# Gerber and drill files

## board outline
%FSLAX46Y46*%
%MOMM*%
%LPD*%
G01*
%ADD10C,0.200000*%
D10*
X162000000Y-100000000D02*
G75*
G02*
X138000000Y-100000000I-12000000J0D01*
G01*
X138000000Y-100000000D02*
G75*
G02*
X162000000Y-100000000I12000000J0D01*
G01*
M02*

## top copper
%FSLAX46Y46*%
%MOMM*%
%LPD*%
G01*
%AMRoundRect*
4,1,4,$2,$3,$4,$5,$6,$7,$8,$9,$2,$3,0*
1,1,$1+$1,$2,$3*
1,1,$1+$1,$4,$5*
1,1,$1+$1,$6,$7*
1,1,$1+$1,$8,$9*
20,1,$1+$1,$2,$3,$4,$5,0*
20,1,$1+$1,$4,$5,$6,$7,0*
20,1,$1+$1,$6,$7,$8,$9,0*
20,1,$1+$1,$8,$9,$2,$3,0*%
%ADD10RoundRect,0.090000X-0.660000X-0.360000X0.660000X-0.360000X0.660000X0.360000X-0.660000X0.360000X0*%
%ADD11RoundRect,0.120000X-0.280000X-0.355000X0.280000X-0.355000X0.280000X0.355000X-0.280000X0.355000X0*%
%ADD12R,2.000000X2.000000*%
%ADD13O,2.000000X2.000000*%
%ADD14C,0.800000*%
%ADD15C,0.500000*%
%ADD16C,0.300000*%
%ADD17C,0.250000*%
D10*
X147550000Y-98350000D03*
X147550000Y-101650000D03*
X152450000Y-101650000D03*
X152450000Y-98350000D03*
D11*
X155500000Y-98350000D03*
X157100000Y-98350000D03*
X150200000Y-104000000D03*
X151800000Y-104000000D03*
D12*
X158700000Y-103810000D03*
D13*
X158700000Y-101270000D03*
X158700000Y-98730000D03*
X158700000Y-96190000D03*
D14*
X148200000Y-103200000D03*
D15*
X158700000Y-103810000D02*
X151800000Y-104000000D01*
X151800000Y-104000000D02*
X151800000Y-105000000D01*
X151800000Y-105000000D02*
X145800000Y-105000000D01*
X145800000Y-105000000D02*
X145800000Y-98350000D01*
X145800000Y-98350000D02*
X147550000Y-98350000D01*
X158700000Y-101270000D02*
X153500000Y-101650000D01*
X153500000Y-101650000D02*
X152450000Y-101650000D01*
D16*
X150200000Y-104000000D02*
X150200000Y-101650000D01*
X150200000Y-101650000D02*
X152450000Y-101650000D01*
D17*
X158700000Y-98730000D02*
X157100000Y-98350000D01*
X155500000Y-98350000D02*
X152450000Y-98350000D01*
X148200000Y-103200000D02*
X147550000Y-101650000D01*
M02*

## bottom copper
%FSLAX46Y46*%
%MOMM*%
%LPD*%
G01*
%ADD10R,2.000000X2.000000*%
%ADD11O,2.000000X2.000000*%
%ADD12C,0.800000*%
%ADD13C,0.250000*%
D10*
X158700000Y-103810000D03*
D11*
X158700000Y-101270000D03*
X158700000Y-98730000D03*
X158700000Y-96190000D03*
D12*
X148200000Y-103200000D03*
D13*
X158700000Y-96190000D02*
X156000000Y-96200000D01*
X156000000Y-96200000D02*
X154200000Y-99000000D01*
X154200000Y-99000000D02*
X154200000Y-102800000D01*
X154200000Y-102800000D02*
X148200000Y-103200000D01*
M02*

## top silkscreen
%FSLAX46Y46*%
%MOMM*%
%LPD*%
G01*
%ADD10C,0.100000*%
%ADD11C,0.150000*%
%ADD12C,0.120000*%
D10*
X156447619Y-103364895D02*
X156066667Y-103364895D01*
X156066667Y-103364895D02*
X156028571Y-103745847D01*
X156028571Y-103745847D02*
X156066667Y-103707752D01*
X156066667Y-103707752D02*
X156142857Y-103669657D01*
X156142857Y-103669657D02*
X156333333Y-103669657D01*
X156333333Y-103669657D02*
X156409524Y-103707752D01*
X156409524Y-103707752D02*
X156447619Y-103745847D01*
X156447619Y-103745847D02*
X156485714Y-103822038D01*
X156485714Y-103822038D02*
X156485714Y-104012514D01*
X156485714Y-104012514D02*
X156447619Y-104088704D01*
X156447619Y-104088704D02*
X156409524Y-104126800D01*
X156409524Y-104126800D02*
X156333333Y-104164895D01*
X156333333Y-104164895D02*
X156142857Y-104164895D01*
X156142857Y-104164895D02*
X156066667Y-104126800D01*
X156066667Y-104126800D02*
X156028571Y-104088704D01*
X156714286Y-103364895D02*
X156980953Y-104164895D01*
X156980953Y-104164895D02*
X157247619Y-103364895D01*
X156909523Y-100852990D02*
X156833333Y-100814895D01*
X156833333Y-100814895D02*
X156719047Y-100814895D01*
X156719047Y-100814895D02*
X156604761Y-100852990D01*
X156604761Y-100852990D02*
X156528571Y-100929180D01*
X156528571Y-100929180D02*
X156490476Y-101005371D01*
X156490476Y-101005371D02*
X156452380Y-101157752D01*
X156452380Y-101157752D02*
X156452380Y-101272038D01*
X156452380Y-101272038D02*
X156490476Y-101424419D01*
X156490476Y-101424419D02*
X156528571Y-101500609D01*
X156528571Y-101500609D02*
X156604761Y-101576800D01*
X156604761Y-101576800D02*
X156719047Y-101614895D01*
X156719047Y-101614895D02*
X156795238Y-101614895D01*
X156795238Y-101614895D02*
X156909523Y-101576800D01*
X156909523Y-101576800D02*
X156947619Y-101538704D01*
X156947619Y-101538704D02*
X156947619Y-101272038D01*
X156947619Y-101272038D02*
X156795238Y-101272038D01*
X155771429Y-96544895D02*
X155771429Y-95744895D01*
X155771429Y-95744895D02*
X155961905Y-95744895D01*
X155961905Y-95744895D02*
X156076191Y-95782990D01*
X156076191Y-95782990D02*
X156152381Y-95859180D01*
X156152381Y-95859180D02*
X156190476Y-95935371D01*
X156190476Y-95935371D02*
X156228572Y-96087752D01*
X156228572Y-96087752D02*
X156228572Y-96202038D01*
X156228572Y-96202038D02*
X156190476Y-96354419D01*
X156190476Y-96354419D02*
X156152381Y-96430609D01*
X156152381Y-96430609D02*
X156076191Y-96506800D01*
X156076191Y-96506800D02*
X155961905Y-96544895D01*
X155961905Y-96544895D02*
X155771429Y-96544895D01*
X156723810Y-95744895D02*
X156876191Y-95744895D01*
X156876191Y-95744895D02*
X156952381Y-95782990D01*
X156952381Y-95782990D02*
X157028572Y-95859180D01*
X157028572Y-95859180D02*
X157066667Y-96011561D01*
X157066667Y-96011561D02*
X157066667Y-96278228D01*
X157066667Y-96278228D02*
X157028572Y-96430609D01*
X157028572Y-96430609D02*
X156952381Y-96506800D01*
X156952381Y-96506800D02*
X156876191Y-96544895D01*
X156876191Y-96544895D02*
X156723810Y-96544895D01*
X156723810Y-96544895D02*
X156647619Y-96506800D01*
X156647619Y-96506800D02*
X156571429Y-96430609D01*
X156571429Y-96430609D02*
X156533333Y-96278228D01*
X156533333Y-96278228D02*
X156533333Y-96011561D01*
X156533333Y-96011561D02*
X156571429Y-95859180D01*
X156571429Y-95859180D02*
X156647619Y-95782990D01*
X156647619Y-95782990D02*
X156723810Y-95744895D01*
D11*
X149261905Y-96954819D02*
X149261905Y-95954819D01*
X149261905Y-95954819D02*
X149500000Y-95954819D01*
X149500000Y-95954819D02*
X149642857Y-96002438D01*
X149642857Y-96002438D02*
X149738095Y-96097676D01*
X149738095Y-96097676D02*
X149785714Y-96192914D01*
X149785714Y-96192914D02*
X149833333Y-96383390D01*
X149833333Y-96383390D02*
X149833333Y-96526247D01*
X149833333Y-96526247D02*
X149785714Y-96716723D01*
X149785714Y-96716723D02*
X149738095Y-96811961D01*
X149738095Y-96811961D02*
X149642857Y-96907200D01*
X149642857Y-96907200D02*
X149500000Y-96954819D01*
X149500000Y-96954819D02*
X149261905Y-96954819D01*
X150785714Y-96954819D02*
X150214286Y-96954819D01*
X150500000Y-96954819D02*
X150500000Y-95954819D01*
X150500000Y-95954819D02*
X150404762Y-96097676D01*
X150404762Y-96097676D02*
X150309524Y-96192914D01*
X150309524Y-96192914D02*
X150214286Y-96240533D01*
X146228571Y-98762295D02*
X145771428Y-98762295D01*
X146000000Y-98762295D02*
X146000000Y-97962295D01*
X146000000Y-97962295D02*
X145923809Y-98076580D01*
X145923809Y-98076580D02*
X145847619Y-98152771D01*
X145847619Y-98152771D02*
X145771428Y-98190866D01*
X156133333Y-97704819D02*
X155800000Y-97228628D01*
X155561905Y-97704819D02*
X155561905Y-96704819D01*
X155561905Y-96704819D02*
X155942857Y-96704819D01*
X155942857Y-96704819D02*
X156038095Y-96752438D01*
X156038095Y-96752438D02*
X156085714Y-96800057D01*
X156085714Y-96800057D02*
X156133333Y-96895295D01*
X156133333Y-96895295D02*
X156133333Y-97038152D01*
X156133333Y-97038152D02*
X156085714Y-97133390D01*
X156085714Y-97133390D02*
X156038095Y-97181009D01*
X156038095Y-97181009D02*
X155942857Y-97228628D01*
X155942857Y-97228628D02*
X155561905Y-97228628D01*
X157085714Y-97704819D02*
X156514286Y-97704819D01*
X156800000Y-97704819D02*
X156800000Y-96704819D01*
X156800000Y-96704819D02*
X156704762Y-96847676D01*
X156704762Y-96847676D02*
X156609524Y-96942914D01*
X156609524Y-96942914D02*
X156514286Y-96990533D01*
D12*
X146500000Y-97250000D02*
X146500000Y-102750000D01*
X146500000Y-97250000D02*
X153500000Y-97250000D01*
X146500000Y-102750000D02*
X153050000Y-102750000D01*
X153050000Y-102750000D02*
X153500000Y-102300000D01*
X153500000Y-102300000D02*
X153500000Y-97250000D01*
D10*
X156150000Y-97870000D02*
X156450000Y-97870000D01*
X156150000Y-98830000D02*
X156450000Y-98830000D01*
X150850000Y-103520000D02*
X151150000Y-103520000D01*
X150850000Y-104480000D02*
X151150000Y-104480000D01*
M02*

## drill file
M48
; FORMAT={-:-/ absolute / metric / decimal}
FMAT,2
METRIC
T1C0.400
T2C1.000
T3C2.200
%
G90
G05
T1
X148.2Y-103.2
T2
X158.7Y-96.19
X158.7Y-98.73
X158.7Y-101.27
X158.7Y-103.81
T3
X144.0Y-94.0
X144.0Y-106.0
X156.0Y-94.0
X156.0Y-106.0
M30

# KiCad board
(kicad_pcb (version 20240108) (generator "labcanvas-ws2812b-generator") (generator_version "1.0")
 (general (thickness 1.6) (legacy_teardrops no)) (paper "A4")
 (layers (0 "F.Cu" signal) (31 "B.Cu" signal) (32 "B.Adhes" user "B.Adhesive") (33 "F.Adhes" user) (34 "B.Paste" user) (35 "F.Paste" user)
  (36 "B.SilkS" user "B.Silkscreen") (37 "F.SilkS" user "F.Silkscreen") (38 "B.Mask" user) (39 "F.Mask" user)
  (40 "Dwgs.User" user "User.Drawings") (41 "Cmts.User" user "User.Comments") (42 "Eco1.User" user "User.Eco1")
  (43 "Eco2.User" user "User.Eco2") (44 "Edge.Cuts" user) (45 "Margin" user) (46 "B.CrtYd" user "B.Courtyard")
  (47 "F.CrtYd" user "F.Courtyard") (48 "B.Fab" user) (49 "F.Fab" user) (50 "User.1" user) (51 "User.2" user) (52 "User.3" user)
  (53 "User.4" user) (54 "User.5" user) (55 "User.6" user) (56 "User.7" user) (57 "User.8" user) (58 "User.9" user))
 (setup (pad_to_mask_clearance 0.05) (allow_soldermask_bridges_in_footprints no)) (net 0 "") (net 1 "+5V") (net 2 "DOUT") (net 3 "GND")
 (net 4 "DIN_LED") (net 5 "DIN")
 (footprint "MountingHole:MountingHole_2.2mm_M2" (layer "F.Cu") (at 144 94)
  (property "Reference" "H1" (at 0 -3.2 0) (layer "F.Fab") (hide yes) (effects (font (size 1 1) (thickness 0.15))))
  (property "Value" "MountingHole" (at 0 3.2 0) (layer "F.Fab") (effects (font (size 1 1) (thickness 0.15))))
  (pad "" np_thru_hole circle (at 0 0) (size 2.2 2.2) (drill 2.2) (layers "*.Cu" "*.Mask")))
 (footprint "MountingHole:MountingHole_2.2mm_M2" (layer "F.Cu") (at 156 94)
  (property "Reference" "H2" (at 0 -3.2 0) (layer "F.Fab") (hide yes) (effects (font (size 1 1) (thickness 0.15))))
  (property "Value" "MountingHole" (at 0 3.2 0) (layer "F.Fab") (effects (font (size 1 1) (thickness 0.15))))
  (pad "" np_thru_hole circle (at 0 0) (size 2.2 2.2) (drill 2.2) (layers "*.Cu" "*.Mask")))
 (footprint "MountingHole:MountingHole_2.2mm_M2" (layer "F.Cu") (at 156 106)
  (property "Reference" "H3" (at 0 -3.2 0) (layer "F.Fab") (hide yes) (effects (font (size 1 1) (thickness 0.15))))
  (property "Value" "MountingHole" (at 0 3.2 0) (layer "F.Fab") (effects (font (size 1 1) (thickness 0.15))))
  (pad "" np_thru_hole circle (at 0 0) (size 2.2 2.2) (drill 2.2) (layers "*.Cu" "*.Mask")))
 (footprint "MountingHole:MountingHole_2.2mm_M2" (layer "F.Cu") (at 144 106)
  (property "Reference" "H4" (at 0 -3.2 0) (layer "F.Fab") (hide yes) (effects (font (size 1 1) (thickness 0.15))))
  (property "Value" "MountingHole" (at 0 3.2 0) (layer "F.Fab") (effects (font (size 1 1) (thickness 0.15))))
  (pad "" np_thru_hole circle (at 0 0) (size 2.2 2.2) (drill 2.2) (layers "*.Cu" "*.Mask")))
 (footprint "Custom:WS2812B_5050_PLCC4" (layer "F.Cu") (at 150 100)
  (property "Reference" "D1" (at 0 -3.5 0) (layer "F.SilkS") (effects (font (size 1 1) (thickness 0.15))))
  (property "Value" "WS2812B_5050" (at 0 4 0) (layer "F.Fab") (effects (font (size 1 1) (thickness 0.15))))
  (fp_line (start -3.5 -2.75) (end -3.5 2.75) (stroke (width 0.12) (type solid)) (layer "F.SilkS"))
  (fp_line (start -3.5 -2.75) (end 3.5 -2.75) (stroke (width 0.12) (type solid)) (layer "F.SilkS"))
  (fp_line (start -3.5 2.75) (end 3.05 2.75) (stroke (width 0.12) (type solid)) (layer "F.SilkS"))
  (fp_line (start 3.05 2.75) (end 3.5 2.3) (stroke (width 0.12) (type solid)) (layer "F.SilkS"))
  (fp_line (start 3.5 2.3) (end 3.5 -2.75) (stroke (width 0.12) (type solid)) (layer "F.SilkS"))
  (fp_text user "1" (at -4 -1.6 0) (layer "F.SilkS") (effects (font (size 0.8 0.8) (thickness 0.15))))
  (pad "1" smd roundrect (at -2.45 -1.65) (size 1.5 0.9) (layers "F.Cu" "F.Mask" "F.Paste") (roundrect_rratio 0.1) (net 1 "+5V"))
  (pad "2" smd roundrect (at -2.45 1.65) (size 1.5 0.9) (layers "F.Cu" "F.Mask" "F.Paste") (roundrect_rratio 0.1) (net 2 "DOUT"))
  (pad "3" smd roundrect (at 2.45 1.65) (size 1.5 0.9) (layers "F.Cu" "F.Mask" "F.Paste") (roundrect_rratio 0.1) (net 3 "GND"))
  (pad "4" smd roundrect (at 2.45 -1.65) (size 1.5 0.9) (layers "F.Cu" "F.Mask" "F.Paste") (roundrect_rratio 0.1) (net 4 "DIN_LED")))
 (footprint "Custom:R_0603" (layer "F.Cu") (at 156.3 98.35)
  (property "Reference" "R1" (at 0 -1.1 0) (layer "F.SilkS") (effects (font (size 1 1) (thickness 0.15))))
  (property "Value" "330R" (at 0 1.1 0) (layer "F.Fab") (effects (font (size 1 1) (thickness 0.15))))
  (fp_line (start -0.15 -0.48) (end 0.15 -0.48) (stroke (width 0.10) (type solid)) (layer "F.SilkS"))
  (fp_line (start -0.15 0.48) (end 0.15 0.48) (stroke (width 0.10) (type solid)) (layer "F.SilkS"))
  (pad "1" smd roundrect (at -0.8 0) (size 0.8 0.95) (layers "F.Cu" "F.Mask" "F.Paste") (roundrect_rratio 0.15) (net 4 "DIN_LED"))
  (pad "2" smd roundrect (at 0.8 0) (size 0.8 0.95) (layers "F.Cu" "F.Mask" "F.Paste") (roundrect_rratio 0.15) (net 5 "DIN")))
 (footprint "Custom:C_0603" (layer "F.Cu") (at 151 104)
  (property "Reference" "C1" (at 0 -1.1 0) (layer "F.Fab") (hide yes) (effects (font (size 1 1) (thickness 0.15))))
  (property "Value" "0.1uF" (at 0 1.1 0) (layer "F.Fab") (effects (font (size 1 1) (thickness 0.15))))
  (fp_line (start -0.15 -0.48) (end 0.15 -0.48) (stroke (width 0.10) (type solid)) (layer "F.SilkS"))
  (fp_line (start -0.15 0.48) (end 0.15 0.48) (stroke (width 0.10) (type solid)) (layer "F.SilkS"))
  (pad "1" smd roundrect (at -0.8 0) (size 0.8 0.95) (layers "F.Cu" "F.Mask" "F.Paste") (roundrect_rratio 0.15) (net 3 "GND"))
  (pad "2" smd roundrect (at 0.8 0) (size 0.8 0.95) (layers "F.Cu" "F.Mask" "F.Paste") (roundrect_rratio 0.15) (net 1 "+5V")))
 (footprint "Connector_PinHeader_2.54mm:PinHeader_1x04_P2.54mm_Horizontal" (layer "B.Cu") (at 158.7 103.81)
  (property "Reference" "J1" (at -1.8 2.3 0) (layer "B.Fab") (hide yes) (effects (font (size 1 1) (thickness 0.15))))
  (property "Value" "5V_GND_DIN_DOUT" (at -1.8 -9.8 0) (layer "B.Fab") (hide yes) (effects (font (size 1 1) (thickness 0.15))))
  (pad "1" thru_hole rect (at 0 0) (size 2.0 2.0) (drill 1.0) (layers "*.Cu" "*.Mask") (remove_unused_layers no) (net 1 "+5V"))
  (pad "2" thru_hole oval (at 0 -2.54) (size 2.0 2.0) (drill 1.0) (layers "*.Cu" "*.Mask") (remove_unused_layers no) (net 3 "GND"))
  (pad "3" thru_hole oval (at 0 -5.08) (size 2.0 2.0) (drill 1.0) (layers "*.Cu" "*.Mask") (remove_unused_layers no) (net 5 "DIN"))
  (pad "4" thru_hole oval (at 0 -7.62) (size 2.0 2.0) (drill 1.0) (layers "*.Cu" "*.Mask") (remove_unused_layers no) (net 2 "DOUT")))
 (gr_circle (center 150 100) (end 162 100) (stroke (width 0.2) (type default)) (fill none) (layer "Edge.Cuts"))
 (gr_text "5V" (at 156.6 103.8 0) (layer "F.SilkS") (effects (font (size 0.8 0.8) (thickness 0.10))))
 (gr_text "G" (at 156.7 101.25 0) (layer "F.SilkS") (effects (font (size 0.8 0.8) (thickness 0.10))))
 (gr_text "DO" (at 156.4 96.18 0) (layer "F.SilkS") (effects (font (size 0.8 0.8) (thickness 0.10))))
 (segment (start 158.7 103.81) (end 151.8 104) (width 0.5) (layer "F.Cu") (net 1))
 (segment (start 151.8 104) (end 151.8 105) (width 0.5) (layer "F.Cu") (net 1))
 (segment (start 151.8 105) (end 145.8 105) (width 0.5) (layer "F.Cu") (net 1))
 (segment (start 145.8 105) (end 145.8 98.35) (width 0.5) (layer "F.Cu") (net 1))
 (segment (start 145.8 98.35) (end 147.55 98.35) (width 0.5) (layer "F.Cu") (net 1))
 (segment (start 158.7 101.27) (end 153.5 101.65) (width 0.5) (layer "F.Cu") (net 3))
 (segment (start 153.5 101.65) (end 152.45 101.65) (width 0.5) (layer "F.Cu") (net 3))
 (segment (start 150.2 104) (end 150.2 101.65) (width 0.3) (layer "F.Cu") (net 3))
 (segment (start 150.2 101.65) (end 152.45 101.65) (width 0.3) (layer "F.Cu") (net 3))
 (segment (start 158.7 98.73) (end 157.1 98.35) (width 0.25) (layer "F.Cu") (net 5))
 (segment (start 155.5 98.35) (end 152.45 98.35) (width 0.25) (layer "F.Cu") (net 4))
 (segment (start 158.7 96.19) (end 156 96.2) (width 0.25) (layer "B.Cu") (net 2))
 (segment (start 156 96.2) (end 154.2 99.0) (width 0.25) (layer "B.Cu") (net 2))
 (segment (start 154.2 99.0) (end 154.2 102.8) (width 0.25) (layer "B.Cu") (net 2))
 (segment (start 154.2 102.8) (end 148.2 103.2) (width 0.25) (layer "B.Cu") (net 2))
 (via (at 148.2 103.2) (size 0.8) (drill 0.4) (layers "F.Cu" "B.Cu") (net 2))
 (segment (start 148.2 103.2) (end 147.55 101.65) (width 0.25) (layer "F.Cu") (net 2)))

